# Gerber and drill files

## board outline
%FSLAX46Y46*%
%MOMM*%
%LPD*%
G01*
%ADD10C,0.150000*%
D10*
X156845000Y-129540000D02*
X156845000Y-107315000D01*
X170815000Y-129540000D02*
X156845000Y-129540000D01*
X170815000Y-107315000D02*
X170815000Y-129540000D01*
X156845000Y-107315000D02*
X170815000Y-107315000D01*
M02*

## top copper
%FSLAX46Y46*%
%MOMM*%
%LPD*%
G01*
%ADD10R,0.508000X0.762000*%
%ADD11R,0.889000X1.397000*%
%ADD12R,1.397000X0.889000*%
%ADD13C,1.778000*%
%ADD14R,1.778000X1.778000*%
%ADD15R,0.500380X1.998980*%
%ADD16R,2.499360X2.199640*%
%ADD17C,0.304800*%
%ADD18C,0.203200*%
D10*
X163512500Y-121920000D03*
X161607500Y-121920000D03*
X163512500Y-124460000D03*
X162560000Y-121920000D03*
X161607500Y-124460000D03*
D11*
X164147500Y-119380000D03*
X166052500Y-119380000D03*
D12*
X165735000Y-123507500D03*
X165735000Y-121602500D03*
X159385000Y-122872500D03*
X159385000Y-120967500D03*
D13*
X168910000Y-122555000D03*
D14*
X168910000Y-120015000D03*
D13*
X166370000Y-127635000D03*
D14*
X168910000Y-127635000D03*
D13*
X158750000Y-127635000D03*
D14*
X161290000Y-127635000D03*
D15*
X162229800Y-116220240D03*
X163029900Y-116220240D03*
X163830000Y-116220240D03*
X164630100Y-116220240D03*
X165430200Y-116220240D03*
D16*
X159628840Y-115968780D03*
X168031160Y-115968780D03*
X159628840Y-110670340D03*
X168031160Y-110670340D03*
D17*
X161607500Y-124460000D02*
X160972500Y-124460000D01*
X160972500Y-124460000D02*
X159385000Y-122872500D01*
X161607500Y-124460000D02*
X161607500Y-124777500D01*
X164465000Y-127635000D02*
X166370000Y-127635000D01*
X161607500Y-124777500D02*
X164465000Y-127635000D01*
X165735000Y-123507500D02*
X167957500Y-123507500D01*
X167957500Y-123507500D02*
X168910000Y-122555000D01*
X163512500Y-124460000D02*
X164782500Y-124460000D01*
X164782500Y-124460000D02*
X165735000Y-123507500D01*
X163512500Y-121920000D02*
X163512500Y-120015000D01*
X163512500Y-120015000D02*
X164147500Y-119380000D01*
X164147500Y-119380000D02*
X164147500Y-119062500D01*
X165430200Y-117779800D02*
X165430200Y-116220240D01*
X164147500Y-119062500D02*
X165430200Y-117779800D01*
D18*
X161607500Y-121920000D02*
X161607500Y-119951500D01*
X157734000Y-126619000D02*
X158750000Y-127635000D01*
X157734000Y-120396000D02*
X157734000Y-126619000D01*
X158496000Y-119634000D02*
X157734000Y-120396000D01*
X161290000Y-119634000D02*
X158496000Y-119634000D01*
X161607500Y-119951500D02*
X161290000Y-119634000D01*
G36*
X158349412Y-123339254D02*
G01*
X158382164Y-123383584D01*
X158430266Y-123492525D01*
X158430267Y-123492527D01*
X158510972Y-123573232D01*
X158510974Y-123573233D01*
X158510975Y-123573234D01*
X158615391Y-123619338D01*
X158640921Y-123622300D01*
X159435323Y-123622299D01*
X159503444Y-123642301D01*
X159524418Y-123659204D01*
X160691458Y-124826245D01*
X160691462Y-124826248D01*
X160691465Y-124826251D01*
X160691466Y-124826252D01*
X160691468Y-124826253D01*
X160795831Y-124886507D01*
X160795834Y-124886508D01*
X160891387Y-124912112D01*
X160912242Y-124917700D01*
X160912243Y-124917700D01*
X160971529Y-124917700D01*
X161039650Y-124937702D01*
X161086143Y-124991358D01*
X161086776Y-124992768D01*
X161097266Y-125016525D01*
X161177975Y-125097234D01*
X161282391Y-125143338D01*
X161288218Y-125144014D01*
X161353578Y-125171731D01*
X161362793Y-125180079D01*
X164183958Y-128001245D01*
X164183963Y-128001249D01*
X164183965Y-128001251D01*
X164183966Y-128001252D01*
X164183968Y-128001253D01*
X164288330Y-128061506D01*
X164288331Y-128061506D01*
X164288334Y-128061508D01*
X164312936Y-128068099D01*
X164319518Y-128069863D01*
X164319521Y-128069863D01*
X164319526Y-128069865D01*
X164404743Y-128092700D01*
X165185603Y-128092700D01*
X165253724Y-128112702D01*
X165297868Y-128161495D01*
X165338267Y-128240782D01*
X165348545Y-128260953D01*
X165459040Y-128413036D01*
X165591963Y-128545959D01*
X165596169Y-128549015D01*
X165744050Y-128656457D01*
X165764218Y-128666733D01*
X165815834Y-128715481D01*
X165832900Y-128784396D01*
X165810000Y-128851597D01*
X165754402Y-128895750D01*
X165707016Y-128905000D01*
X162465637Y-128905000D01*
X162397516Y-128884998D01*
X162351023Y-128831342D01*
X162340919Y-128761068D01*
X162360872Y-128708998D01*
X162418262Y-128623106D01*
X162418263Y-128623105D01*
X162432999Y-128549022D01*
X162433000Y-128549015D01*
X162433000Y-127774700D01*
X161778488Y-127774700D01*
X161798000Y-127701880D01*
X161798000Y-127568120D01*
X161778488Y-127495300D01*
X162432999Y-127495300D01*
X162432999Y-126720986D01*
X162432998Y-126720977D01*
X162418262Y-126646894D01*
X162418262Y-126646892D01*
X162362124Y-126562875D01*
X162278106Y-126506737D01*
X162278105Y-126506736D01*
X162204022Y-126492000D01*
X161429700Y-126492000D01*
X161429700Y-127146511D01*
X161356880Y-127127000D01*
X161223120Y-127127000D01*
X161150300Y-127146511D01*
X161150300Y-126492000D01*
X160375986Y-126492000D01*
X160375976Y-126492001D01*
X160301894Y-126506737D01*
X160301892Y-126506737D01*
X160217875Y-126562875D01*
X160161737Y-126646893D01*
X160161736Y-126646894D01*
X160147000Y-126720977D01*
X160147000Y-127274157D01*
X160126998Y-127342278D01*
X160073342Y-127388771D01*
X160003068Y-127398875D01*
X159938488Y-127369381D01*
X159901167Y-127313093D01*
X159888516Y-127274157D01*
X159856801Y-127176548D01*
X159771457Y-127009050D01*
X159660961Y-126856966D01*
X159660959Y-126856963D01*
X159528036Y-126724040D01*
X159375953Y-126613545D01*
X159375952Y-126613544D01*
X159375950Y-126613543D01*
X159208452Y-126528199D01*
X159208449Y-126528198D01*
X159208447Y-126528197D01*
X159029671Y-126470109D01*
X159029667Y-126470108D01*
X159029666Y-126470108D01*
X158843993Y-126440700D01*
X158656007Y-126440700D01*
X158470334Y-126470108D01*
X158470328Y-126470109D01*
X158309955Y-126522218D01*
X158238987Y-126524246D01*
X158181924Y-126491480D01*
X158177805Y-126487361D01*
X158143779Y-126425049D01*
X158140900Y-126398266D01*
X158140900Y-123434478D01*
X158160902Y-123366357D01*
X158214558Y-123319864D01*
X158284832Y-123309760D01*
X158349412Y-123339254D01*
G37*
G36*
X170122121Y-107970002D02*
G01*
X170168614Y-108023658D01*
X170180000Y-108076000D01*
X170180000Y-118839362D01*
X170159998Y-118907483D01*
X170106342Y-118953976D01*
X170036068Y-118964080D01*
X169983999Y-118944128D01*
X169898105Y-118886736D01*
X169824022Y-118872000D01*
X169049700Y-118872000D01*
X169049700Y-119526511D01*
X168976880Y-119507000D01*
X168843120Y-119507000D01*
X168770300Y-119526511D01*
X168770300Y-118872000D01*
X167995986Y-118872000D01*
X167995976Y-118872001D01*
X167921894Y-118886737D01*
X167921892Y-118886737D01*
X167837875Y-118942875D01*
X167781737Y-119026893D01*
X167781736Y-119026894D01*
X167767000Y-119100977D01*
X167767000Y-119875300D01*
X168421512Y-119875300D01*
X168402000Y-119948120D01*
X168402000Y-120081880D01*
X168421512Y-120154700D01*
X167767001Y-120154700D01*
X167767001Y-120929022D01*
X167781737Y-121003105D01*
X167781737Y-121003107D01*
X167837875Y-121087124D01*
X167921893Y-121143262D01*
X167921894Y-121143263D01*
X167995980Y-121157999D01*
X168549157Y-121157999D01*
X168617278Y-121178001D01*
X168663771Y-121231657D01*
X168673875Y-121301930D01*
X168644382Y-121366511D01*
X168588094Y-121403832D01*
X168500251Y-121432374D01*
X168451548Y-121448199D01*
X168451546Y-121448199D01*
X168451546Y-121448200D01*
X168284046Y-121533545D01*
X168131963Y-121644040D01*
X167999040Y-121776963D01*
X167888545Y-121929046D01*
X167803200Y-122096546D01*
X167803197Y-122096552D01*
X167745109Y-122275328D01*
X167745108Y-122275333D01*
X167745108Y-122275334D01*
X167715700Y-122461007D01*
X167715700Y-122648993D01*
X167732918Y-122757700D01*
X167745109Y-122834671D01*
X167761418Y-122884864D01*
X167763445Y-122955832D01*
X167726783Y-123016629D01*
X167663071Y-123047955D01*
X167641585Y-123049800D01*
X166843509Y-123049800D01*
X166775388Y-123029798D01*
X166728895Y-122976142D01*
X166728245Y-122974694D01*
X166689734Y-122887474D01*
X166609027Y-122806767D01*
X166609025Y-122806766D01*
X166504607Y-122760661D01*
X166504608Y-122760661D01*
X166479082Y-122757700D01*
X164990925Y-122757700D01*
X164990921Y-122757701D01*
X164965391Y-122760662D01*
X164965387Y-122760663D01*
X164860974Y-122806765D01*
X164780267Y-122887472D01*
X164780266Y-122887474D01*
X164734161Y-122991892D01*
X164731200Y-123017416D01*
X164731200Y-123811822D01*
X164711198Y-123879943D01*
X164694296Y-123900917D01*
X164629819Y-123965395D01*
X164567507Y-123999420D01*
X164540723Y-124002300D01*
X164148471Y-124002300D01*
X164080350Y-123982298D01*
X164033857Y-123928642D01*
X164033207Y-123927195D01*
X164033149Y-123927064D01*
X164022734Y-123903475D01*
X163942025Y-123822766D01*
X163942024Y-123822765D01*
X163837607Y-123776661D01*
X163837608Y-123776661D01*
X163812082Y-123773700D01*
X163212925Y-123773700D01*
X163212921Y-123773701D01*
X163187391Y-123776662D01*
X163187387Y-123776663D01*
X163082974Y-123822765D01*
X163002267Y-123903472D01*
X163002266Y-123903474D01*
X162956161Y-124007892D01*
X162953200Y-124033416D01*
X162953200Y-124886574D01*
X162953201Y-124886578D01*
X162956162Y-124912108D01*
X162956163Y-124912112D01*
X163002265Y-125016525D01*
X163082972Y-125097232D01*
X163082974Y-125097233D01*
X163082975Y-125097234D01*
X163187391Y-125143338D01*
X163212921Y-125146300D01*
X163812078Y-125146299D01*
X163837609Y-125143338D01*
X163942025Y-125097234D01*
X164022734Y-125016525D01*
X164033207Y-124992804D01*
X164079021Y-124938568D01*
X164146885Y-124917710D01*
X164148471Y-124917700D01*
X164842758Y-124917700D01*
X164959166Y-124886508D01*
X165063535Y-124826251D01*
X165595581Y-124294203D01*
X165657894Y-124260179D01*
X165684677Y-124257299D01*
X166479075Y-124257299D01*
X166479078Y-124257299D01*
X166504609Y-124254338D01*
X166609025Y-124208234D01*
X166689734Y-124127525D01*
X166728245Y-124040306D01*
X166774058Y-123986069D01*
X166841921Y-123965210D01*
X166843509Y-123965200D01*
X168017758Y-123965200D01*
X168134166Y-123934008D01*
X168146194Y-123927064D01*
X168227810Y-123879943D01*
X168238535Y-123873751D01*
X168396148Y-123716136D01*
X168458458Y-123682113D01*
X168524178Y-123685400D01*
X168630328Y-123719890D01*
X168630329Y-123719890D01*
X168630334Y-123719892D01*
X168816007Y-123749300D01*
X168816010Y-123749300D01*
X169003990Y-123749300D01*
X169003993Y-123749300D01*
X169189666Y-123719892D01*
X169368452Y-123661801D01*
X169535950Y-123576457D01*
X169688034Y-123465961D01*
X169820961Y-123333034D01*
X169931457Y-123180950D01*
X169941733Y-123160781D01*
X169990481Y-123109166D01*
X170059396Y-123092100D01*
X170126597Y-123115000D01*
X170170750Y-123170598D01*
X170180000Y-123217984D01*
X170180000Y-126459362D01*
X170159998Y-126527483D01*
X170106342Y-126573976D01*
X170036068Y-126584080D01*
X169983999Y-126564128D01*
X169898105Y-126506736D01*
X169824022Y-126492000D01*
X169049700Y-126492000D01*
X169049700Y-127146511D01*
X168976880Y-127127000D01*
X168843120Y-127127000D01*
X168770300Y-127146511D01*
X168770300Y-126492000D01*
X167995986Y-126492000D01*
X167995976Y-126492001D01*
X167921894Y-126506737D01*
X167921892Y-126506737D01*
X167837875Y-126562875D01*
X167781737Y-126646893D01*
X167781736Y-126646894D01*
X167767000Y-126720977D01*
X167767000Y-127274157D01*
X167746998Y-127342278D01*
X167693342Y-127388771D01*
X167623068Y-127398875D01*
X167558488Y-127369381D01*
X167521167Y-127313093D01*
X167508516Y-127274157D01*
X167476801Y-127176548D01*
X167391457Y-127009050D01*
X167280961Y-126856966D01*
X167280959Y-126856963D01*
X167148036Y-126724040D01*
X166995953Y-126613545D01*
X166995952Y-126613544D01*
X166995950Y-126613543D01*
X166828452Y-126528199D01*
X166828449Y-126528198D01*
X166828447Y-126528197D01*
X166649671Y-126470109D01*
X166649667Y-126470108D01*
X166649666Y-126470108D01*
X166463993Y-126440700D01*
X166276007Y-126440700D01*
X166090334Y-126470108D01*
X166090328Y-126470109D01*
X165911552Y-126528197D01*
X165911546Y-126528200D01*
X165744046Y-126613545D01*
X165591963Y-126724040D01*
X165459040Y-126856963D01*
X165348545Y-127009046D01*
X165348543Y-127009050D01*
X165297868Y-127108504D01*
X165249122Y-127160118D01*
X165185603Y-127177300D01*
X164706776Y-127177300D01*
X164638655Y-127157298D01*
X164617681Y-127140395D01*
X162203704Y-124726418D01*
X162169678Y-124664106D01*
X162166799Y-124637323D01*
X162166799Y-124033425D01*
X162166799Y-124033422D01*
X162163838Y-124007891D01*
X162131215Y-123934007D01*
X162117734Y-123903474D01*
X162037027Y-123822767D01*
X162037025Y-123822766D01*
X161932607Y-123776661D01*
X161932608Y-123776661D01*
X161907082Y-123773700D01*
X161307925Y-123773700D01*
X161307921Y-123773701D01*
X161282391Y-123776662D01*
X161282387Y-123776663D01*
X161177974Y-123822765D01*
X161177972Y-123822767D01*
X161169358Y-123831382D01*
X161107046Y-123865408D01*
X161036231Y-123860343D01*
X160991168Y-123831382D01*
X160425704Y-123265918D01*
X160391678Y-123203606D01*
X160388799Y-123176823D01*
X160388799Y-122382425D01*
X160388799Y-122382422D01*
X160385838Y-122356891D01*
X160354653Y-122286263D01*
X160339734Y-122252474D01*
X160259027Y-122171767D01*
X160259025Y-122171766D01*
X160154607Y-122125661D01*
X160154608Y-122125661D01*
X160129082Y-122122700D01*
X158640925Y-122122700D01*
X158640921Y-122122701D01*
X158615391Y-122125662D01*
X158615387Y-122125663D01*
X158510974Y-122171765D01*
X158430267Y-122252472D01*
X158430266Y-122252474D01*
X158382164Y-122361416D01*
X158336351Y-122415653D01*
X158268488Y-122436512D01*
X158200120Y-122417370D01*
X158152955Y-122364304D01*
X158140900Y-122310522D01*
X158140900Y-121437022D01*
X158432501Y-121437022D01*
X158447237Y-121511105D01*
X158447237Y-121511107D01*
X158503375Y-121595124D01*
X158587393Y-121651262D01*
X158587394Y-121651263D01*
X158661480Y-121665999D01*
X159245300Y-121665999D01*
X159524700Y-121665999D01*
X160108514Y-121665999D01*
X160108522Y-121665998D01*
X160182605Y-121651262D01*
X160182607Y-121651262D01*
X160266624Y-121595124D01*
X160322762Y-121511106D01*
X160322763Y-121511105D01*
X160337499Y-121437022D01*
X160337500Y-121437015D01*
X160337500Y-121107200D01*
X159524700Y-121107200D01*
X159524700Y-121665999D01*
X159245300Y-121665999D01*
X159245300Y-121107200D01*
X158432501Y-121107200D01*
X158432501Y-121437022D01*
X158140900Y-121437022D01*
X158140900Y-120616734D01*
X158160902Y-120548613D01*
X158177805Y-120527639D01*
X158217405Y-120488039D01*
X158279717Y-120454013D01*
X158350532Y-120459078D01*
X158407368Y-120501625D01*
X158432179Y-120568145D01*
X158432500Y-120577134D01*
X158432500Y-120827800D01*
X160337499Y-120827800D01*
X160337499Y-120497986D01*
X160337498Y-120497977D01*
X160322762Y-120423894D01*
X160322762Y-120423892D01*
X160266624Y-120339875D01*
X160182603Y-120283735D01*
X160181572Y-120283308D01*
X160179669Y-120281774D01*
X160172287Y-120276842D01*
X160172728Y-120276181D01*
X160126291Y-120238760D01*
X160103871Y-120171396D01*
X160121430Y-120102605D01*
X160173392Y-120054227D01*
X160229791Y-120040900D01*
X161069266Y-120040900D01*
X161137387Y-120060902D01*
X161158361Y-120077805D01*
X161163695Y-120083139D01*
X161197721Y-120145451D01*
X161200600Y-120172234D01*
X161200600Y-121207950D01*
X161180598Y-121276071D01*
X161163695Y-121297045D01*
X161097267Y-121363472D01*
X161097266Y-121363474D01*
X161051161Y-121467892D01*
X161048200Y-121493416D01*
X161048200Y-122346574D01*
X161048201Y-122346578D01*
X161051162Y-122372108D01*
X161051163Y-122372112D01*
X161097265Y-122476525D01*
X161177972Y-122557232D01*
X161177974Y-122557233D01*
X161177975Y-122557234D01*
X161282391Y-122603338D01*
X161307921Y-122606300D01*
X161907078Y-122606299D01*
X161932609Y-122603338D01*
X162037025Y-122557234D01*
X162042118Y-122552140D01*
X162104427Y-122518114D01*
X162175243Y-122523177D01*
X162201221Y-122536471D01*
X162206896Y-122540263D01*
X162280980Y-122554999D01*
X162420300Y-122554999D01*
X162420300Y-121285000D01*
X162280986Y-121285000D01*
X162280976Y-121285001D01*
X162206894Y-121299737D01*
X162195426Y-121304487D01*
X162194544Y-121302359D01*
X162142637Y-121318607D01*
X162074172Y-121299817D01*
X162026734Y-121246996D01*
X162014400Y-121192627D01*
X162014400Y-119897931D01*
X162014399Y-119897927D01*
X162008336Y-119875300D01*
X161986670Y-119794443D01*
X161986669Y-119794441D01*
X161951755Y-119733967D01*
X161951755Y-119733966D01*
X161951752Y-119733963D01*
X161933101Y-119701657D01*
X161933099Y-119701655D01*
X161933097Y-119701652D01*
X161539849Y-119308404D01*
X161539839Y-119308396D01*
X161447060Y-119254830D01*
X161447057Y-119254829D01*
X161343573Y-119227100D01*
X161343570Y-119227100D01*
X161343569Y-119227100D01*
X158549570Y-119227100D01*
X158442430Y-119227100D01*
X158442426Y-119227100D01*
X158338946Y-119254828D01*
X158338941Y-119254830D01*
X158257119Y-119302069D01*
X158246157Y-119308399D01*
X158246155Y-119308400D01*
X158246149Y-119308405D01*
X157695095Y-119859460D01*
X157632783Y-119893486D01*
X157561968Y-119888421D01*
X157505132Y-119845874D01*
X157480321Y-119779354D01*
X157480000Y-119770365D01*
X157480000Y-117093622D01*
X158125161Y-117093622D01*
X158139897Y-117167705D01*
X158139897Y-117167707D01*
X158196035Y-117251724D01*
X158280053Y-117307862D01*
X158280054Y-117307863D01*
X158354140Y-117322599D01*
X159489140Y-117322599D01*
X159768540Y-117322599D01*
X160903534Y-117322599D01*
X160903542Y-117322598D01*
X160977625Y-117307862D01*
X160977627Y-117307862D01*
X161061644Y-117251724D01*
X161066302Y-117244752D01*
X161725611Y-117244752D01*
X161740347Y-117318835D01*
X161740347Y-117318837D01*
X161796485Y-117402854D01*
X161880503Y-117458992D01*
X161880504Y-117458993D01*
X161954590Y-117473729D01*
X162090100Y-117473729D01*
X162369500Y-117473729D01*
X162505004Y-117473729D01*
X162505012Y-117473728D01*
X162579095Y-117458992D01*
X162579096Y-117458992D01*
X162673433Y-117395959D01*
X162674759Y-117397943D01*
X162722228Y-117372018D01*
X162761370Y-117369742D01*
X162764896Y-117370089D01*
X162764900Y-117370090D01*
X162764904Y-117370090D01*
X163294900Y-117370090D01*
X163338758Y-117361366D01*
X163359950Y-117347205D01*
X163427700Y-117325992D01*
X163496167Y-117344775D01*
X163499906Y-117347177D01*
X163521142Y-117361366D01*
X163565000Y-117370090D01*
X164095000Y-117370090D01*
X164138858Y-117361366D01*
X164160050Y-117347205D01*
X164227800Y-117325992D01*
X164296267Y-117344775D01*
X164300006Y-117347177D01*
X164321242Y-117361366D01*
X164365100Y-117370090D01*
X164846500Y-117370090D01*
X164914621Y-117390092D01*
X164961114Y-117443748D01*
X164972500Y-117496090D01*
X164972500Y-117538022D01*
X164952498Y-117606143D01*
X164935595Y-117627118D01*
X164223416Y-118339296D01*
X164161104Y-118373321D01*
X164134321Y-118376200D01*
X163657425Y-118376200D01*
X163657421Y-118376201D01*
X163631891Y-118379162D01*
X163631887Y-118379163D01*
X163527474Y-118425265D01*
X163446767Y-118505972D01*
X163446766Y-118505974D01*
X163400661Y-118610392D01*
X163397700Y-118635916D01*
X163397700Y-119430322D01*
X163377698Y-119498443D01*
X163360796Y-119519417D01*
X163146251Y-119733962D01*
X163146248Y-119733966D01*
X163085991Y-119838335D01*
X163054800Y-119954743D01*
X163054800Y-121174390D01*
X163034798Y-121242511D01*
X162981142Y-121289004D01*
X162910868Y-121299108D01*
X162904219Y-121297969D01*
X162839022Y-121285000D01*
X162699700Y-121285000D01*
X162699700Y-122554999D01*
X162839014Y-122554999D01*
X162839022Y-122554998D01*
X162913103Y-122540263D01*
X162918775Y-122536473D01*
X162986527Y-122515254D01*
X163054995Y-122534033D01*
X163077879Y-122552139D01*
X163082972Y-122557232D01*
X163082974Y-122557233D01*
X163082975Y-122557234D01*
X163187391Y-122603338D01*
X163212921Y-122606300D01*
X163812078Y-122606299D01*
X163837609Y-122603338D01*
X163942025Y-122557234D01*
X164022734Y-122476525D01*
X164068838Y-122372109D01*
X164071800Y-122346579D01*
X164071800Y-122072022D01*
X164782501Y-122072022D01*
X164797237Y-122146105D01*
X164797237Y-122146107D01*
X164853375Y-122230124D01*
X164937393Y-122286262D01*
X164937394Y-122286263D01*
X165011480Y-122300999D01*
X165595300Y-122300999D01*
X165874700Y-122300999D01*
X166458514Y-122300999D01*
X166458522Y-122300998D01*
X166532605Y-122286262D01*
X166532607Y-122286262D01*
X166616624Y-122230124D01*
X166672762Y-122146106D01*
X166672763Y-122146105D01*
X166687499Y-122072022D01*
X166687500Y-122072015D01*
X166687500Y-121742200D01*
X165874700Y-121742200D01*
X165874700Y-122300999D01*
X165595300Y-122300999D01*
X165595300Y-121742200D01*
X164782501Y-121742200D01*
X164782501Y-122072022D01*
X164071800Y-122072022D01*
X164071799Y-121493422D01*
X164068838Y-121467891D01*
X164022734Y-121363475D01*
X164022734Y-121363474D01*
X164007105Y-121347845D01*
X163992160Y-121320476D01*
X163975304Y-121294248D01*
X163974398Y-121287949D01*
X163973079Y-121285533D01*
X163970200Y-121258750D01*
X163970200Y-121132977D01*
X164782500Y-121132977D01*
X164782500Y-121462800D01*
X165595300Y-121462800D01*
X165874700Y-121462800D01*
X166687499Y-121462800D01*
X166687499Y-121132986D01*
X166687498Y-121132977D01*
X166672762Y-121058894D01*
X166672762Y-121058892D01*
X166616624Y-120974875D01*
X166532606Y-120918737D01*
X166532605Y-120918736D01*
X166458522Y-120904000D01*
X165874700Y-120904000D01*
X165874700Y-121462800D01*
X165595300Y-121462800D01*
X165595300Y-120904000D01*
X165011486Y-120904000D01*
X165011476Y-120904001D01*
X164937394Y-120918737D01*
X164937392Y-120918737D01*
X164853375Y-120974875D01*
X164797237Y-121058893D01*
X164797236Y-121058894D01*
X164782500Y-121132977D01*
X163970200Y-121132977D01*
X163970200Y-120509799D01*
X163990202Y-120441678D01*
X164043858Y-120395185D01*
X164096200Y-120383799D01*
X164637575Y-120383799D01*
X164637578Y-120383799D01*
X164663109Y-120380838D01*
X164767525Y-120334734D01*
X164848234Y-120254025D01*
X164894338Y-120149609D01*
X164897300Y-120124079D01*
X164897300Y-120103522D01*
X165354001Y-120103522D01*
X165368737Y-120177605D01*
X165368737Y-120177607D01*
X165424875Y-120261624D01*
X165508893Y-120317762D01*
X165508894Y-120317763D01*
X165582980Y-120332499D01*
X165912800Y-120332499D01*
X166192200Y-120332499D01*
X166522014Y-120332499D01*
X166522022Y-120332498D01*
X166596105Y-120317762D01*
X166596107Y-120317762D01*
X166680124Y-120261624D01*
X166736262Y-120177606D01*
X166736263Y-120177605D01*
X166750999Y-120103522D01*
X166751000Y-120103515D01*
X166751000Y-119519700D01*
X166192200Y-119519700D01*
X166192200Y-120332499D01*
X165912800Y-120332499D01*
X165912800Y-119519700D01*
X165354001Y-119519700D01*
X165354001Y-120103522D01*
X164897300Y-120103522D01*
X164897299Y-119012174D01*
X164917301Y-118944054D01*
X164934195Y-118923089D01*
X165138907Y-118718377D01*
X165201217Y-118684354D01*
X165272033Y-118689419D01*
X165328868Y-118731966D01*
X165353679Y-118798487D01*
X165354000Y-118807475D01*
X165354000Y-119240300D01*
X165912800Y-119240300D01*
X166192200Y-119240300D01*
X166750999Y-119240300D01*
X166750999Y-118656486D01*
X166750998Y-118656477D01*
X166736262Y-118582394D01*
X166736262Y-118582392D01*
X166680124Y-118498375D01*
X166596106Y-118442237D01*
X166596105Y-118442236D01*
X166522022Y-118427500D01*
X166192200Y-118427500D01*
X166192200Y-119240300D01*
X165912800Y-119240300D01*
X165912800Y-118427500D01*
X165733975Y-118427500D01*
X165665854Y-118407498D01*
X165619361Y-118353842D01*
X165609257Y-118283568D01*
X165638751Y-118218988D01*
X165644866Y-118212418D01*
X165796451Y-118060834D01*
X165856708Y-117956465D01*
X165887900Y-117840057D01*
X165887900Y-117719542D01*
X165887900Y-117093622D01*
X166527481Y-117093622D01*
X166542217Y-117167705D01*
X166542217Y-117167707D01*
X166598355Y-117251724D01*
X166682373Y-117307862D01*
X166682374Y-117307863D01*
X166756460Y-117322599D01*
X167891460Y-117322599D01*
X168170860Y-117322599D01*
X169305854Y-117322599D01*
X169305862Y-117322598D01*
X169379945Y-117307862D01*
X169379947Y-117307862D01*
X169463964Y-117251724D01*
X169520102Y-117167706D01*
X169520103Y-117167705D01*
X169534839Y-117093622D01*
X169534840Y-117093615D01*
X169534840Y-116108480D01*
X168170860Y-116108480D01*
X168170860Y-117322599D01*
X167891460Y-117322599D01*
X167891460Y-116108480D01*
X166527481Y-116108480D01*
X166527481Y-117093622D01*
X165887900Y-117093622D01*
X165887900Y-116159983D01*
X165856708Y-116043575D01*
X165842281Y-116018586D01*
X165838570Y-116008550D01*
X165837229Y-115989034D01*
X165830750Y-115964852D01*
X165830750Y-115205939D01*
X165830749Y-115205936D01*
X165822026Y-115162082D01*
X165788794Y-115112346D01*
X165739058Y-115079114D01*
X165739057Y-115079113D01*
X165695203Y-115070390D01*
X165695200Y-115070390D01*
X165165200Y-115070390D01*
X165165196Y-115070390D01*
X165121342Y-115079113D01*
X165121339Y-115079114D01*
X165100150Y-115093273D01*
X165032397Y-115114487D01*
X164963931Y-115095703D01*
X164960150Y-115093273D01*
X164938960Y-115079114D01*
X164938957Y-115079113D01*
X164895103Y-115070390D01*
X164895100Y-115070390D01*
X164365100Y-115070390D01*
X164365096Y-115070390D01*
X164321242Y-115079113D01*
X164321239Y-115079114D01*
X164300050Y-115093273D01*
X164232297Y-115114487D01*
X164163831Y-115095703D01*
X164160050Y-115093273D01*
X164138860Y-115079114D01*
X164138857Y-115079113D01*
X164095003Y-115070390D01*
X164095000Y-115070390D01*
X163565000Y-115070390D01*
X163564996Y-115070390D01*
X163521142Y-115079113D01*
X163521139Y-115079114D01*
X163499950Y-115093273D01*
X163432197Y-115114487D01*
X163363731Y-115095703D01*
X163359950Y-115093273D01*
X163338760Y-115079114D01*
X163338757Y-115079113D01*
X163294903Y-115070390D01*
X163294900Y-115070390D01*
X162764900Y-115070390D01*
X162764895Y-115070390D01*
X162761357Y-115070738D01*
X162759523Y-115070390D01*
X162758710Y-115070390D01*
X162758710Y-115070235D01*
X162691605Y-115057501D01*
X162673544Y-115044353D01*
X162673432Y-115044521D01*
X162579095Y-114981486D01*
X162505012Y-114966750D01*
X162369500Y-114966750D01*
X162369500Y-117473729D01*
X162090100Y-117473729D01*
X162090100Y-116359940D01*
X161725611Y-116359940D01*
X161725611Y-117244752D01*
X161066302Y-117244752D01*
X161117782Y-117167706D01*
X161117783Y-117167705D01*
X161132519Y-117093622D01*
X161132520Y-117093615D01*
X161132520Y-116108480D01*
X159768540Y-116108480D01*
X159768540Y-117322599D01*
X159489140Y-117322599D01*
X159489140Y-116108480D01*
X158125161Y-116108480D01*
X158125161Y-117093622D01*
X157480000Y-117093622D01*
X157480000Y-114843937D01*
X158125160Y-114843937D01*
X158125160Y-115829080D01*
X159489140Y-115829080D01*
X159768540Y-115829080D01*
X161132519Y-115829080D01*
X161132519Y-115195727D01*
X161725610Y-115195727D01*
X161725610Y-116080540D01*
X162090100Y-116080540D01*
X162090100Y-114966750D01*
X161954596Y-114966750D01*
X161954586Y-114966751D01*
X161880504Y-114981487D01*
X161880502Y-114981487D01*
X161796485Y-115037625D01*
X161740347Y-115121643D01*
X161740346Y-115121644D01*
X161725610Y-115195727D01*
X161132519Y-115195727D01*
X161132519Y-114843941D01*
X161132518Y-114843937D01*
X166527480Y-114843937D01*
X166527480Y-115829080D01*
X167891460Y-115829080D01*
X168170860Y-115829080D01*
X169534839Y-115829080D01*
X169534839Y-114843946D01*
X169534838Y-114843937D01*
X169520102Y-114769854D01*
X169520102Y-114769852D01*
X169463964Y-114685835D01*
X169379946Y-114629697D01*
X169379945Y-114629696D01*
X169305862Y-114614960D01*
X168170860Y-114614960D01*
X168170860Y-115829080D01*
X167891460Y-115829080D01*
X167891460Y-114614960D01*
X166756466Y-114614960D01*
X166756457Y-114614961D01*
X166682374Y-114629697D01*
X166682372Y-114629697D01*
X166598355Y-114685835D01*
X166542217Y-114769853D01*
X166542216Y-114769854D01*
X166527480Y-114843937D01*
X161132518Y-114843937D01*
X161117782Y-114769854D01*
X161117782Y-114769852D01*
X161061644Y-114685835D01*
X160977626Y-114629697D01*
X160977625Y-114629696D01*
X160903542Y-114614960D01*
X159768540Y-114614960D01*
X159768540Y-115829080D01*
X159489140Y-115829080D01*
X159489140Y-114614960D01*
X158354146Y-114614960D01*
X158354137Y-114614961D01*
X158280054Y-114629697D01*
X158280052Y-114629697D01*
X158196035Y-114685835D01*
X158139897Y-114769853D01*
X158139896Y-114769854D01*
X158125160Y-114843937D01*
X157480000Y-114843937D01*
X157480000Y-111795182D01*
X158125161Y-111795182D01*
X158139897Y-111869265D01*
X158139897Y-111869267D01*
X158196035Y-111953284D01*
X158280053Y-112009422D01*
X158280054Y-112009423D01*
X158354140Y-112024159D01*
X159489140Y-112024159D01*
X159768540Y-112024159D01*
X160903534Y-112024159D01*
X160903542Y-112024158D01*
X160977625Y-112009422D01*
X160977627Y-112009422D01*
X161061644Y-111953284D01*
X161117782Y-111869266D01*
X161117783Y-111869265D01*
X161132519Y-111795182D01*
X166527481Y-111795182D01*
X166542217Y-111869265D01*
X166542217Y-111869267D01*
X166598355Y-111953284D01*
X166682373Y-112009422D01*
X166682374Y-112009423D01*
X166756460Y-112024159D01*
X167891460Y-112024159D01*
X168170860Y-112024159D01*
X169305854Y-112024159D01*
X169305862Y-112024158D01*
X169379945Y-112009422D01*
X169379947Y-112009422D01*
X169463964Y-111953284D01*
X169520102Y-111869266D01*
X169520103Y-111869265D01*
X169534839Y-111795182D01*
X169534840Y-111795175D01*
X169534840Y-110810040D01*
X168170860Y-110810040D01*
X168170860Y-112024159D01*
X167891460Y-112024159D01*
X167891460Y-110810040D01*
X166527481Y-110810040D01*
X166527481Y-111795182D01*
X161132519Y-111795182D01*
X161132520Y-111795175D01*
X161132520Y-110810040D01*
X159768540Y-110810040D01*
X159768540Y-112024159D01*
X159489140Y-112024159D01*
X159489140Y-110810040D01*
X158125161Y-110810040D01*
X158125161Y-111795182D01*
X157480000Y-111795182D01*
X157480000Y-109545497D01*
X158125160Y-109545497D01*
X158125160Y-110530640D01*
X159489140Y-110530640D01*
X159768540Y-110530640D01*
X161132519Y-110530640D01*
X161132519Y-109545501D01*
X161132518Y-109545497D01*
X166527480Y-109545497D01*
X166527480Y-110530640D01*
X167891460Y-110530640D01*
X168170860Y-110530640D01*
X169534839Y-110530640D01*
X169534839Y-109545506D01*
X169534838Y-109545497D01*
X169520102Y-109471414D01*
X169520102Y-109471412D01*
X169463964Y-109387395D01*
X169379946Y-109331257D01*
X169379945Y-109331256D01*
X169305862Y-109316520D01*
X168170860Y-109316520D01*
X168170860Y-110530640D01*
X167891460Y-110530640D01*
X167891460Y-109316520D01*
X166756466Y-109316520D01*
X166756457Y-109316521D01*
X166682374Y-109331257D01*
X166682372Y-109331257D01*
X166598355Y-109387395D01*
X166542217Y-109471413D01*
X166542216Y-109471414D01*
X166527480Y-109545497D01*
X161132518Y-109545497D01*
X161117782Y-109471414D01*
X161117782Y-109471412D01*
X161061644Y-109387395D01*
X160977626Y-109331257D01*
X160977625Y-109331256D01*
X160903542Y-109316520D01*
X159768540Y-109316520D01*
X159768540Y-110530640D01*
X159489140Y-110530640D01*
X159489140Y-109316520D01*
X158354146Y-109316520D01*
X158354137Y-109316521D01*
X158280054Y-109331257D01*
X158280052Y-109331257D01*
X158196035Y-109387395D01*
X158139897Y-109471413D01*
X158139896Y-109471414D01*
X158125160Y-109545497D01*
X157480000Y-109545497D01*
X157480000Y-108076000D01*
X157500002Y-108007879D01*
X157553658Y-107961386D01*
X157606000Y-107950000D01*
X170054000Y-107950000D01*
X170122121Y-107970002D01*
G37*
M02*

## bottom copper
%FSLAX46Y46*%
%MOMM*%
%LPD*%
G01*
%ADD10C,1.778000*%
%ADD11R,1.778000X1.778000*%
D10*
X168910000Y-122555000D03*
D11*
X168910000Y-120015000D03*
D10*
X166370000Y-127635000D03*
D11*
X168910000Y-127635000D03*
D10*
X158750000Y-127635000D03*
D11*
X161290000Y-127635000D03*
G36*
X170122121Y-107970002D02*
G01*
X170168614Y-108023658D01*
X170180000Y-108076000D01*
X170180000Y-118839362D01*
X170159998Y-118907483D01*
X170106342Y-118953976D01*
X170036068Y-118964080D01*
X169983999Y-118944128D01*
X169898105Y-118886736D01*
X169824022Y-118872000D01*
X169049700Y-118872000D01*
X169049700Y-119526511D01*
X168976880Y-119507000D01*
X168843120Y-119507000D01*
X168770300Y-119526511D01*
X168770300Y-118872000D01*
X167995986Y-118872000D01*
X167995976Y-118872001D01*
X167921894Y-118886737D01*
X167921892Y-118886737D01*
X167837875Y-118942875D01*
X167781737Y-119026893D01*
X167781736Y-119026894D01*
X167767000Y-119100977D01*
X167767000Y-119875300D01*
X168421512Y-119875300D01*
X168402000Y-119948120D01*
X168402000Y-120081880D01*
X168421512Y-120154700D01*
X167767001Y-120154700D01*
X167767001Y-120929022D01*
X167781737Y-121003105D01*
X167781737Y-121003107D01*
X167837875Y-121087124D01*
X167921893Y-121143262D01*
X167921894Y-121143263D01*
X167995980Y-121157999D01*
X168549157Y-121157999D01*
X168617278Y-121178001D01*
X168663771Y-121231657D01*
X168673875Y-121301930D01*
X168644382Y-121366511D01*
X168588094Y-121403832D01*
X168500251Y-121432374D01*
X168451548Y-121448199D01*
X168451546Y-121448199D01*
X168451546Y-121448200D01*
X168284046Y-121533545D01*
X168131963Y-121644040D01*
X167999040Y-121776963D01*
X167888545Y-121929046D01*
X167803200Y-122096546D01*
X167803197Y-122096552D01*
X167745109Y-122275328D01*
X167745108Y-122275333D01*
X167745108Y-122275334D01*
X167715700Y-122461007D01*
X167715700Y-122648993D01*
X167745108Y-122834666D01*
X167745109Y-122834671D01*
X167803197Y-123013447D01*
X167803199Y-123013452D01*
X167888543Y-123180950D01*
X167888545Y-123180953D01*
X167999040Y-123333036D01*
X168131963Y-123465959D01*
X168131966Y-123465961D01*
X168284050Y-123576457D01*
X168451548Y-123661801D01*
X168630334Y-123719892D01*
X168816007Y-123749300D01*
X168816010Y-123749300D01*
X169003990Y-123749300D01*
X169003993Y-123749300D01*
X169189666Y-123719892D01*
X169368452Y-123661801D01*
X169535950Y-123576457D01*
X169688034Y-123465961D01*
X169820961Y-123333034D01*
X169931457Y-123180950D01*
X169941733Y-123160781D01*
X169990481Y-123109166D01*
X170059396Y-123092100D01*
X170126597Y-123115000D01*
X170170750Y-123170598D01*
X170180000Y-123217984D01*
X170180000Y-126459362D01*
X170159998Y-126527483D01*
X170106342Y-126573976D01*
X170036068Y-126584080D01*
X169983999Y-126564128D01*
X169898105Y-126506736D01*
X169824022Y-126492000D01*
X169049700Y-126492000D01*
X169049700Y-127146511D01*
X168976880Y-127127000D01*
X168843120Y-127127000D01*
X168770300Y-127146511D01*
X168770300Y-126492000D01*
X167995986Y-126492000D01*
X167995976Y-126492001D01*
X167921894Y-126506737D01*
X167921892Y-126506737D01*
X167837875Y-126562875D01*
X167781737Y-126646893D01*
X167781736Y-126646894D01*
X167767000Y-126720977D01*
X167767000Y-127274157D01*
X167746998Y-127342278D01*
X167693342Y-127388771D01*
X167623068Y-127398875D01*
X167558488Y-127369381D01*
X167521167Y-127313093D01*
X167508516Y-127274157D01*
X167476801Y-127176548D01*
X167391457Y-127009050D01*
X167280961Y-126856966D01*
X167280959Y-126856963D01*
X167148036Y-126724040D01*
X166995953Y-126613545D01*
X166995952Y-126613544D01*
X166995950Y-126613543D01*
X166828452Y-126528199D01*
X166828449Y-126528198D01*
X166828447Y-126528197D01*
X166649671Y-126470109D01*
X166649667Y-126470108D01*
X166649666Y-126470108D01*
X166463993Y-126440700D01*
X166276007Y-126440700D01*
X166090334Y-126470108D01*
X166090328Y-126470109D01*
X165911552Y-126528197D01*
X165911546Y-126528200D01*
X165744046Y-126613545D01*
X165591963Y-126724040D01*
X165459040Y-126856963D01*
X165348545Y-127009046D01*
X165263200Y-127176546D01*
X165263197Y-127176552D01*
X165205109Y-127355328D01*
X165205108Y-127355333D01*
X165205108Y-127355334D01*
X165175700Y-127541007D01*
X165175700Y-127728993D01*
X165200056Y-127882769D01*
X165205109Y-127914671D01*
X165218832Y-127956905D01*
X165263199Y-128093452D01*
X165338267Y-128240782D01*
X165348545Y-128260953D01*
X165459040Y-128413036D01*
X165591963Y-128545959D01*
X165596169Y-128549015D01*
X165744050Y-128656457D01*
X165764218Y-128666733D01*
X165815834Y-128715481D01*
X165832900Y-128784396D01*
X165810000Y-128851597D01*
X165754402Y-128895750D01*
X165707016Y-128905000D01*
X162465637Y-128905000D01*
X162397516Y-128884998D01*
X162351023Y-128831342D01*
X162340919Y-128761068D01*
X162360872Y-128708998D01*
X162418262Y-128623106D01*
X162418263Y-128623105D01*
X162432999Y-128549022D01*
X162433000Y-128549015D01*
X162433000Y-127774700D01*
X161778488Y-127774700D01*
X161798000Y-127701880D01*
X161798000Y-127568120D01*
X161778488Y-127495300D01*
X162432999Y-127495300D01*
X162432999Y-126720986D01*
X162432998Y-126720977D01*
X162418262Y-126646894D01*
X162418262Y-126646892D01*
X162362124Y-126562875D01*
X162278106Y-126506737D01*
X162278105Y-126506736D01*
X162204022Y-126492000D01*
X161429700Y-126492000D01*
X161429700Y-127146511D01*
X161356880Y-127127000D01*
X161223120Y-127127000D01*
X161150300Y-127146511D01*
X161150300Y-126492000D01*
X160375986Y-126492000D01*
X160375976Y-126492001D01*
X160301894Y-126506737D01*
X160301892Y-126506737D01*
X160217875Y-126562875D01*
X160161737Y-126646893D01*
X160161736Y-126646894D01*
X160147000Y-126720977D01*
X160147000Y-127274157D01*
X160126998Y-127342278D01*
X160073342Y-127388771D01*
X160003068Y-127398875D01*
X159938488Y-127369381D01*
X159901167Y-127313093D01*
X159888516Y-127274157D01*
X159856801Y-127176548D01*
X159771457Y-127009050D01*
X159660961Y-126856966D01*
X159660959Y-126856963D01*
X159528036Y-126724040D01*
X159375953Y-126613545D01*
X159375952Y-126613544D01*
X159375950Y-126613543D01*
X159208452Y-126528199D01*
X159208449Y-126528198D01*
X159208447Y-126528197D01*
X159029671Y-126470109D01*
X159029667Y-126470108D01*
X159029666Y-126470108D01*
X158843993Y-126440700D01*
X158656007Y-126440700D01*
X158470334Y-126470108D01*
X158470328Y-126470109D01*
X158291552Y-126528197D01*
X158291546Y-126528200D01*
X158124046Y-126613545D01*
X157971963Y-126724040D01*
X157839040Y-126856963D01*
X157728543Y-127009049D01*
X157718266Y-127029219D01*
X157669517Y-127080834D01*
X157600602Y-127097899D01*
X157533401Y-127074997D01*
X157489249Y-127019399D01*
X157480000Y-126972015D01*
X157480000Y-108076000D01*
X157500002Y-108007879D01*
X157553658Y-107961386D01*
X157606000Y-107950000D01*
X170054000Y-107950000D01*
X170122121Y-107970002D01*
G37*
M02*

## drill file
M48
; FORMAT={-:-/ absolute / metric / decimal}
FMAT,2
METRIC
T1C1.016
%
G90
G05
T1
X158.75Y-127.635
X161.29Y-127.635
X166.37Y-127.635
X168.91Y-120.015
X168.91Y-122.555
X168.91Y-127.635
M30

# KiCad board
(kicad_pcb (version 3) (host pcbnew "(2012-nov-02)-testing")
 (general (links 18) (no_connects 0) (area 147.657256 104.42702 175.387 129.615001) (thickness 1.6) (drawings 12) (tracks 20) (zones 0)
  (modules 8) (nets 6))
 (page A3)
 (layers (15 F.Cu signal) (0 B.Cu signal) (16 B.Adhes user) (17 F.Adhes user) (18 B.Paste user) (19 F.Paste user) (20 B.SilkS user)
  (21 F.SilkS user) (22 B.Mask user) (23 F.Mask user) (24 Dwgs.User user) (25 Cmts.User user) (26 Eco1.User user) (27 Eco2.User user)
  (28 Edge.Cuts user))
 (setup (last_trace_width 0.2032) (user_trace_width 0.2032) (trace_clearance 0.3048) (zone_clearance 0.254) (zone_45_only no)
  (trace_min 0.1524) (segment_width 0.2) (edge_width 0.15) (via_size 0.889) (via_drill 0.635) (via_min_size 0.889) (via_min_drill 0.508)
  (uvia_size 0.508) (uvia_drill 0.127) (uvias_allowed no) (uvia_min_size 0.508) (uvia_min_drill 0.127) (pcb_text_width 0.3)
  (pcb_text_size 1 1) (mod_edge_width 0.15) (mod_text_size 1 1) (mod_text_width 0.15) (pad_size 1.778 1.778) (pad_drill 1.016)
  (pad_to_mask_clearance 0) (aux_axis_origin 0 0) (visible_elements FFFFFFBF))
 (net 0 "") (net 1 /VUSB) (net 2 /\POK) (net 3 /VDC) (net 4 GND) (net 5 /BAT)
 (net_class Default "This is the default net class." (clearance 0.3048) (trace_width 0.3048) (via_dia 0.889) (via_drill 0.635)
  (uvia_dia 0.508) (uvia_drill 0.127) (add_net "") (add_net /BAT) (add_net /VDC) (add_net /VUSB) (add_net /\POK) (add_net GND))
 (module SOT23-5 (layer F.Cu) (at 162.56 123.19 180)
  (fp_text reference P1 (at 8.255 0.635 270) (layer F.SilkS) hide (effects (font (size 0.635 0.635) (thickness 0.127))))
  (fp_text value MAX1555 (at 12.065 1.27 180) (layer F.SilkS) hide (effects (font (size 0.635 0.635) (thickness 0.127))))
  (pad 1 smd rect (at -0.9525 1.27 180) (size 0.508 0.762) (layers F.Cu F.Paste F.Mask) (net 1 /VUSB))
  (pad 3 smd rect (at 0.9525 1.27 180) (size 0.508 0.762) (layers F.Cu F.Paste F.Mask) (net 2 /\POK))
  (pad 5 smd rect (at -0.9525 -1.27 180) (size 0.508 0.762) (layers F.Cu F.Paste F.Mask) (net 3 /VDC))
  (pad 2 smd rect (at 0 1.27 180) (size 0.508 0.762) (layers F.Cu F.Paste F.Mask) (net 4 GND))
  (pad 4 smd rect (at 0.9525 -1.27 180) (size 0.508 0.762) (layers F.Cu F.Paste F.Mask) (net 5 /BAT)))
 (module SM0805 (layer F.Cu) (at 165.1 119.38)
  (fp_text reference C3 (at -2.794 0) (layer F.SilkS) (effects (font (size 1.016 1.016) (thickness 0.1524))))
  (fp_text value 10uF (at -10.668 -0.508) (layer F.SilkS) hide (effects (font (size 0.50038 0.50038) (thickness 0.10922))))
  (pad 1 smd rect (at -0.9525 0) (size 0.889 1.397) (layers F.Cu F.Paste F.Mask) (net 1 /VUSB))
  (pad 2 smd rect (at 0.9525 0) (size 0.889 1.397) (layers F.Cu F.Paste F.Mask) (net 4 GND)))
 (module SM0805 (layer F.Cu) (at 165.735 122.555 90)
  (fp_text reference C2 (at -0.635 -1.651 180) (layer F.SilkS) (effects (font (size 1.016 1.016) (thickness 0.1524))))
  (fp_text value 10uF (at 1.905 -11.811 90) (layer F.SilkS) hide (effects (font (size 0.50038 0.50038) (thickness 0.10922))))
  (pad 1 smd rect (at -0.9525 0 90) (size 0.889 1.397) (layers F.Cu F.Paste F.Mask) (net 3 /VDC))
  (pad 2 smd rect (at 0.9525 0 90) (size 0.889 1.397) (layers F.Cu F.Paste F.Mask) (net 4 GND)))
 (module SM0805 (layer F.Cu) (at 159.385 121.92 90)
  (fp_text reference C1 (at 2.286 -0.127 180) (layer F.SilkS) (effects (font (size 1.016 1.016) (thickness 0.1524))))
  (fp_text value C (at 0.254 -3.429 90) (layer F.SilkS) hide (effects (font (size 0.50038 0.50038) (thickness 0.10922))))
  (pad 1 smd rect (at -0.9525 0 90) (size 0.889 1.397) (layers F.Cu F.Paste F.Mask) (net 5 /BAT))
  (pad 2 smd rect (at 0.9525 0 90) (size 0.889 1.397) (layers F.Cu F.Paste F.Mask) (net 4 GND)))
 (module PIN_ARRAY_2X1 (layer F.Cu) (at 168.91 121.285 90)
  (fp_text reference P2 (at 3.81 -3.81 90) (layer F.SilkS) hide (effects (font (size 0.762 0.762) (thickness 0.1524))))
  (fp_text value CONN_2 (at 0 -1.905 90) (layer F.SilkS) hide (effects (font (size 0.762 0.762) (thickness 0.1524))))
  (pad 1 thru_hole circle (at -1.27 0 90) (size 1.778 1.778) (drill 1.016) (layers *.Cu *.Mask F.SilkS) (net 3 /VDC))
  (pad 2 thru_hole rect (at 1.27 0 90) (size 1.778 1.778) (drill 1.016) (layers *.Cu *.Mask F.SilkS) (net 4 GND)))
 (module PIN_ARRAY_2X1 (layer F.Cu) (at 167.64 127.635)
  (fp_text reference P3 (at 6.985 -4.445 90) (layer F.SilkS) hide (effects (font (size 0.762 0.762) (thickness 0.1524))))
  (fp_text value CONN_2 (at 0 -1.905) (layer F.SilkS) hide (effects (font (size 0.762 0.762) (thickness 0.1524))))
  (pad 1 thru_hole circle (at -1.27 0) (size 1.778 1.778) (drill 1.016) (layers *.Cu *.Mask F.SilkS) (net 5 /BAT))
  (pad 2 thru_hole rect (at 1.27 0) (size 1.778 1.778) (drill 1.016) (layers *.Cu *.Mask F.SilkS) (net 4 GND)))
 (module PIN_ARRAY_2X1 (layer F.Cu) (at 160.02 127.635)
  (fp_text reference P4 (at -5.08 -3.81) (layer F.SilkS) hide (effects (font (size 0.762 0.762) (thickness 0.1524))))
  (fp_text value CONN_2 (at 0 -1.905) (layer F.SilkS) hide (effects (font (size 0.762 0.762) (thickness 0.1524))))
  (pad 1 thru_hole circle (at -1.27 0) (size 1.778 1.778) (drill 1.016) (layers *.Cu *.Mask F.SilkS) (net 2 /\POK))
  (pad 2 thru_hole rect (at 1.27 0) (size 1.778 1.778) (drill 1.016) (layers *.Cu *.Mask F.SilkS) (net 4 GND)))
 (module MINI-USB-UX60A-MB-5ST (layer F.Cu) (at 163.83 112.395 180)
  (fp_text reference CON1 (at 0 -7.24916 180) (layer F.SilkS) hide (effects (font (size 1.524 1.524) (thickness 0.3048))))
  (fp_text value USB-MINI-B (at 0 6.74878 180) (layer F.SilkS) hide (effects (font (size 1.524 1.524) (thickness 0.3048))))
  (pad 5 smd rect (at 1.6002 -3.82524 180) (size 0.50038 1.99898) (layers F.Cu F.Paste F.Mask) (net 4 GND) (clearance 0.14986))
  (pad 4 smd rect (at 0.8001 -3.82524 180) (size 0.50038 1.99898) (layers F.Cu F.Paste F.Mask) (clearance 0.14986))
  (pad 3 smd rect (at 0 -3.82524 180) (size 0.50038 1.99898) (layers F.Cu F.Paste F.Mask) (clearance 0.14986))
  (pad 2 smd rect (at -0.8001 -3.82524 180) (size 0.50038 1.99898) (layers F.Cu F.Paste F.Mask) (clearance 0.14986))
  (pad 1 smd rect (at -1.6002 -3.82524 180) (size 0.50038 1.99898) (layers F.Cu F.Paste F.Mask) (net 1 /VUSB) (clearance 0.14986))
  (pad 6 smd rect (at 4.20116 -3.57378 180) (size 2.49936 2.19964) (layers F.Cu F.Paste F.Mask) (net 4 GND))
  (pad 6 smd rect (at -4.20116 -3.57378 180) (size 2.49936 2.19964) (layers F.Cu F.Paste F.Mask) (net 4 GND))
  (pad 6 smd rect (at 4.20116 1.72466 180) (size 2.49936 2.19964) (layers F.Cu F.Paste F.Mask) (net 4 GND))
  (pad 6 smd rect (at -4.20116 1.72466 180) (size 2.49936 2.19964) (layers F.Cu F.Paste F.Mask) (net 4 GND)))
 (gr_line (start 156.845 129.54) (end 156.845 107.315) (angle 90) (layer Edge.Cuts) (width 0.15))
 (gr_line (start 170.815 129.54) (end 156.845 129.54) (angle 90) (layer Edge.Cuts) (width 0.15))
 (gr_line (start 170.815 107.315) (end 170.815 129.54) (angle 90) (layer Edge.Cuts) (width 0.15))
 (gr_line (start 156.845 107.315) (end 170.815 107.315) (angle 90) (layer Edge.Cuts) (width 0.15))
 (segment (start 161.6075 124.46) (end 160.9725 124.46) (width 0.3048) (layer F.Cu) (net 5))
 (segment (start 160.9725 124.46) (end 159.385 122.8725) (width 0.3048) (layer F.Cu) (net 5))
 (segment (start 161.6075 124.46) (end 161.6075 124.7775) (width 0.3048) (layer F.Cu) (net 5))
 (segment (start 164.465 127.635) (end 166.37 127.635) (width 0.3048) (layer F.Cu) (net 5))
 (segment (start 161.6075 124.7775) (end 164.465 127.635) (width 0.3048) (layer F.Cu) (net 5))
 (segment (start 165.735 123.5075) (end 167.9575 123.5075) (width 0.3048) (layer F.Cu) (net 3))
 (segment (start 167.9575 123.5075) (end 168.91 122.555) (width 0.3048) (layer F.Cu) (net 3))
 (segment (start 163.5125 124.46) (end 164.7825 124.46) (width 0.3048) (layer F.Cu) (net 3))
 (segment (start 164.7825 124.46) (end 165.735 123.5075) (width 0.3048) (layer F.Cu) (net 3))
 (segment (start 163.5125 121.92) (end 163.5125 120.015) (width 0.3048) (layer F.Cu) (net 1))
 (segment (start 163.5125 120.015) (end 164.1475 119.38) (width 0.3048) (layer F.Cu) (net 1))
 (segment (start 164.1475 119.38) (end 164.1475 119.0625) (width 0.3048) (layer F.Cu) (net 1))
 (segment (start 165.4302 117.7798) (end 165.4302 116.22024) (width 0.3048) (layer F.Cu) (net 1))
 (segment (start 164.1475 119.0625) (end 165.4302 117.7798) (width 0.3048) (layer F.Cu) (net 1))
 (segment (start 161.6075 121.92) (end 161.6075 119.9515) (width 0.2032) (layer F.Cu) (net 2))
 (segment (start 157.734 126.619) (end 158.75 127.635) (width 0.2032) (layer F.Cu) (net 2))
 (segment (start 157.734 120.396) (end 157.734 126.619) (width 0.2032) (layer F.Cu) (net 2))
 (segment (start 158.496 119.634) (end 157.734 120.396) (width 0.2032) (layer F.Cu) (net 2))
 (segment (start 161.29 119.634) (end 158.496 119.634) (width 0.2032) (layer F.Cu) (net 2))
 (segment (start 161.6075 119.9515) (end 161.29 119.634) (width 0.2032) (layer F.Cu) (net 2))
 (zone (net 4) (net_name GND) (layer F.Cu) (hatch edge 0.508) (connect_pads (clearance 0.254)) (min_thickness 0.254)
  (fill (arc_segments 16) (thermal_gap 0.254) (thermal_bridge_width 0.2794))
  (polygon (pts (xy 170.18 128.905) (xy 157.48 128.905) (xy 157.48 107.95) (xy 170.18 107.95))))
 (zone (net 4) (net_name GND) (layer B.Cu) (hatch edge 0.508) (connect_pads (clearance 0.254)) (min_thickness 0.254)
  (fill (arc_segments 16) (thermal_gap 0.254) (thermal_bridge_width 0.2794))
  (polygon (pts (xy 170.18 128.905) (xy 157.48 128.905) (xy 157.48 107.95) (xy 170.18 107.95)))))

